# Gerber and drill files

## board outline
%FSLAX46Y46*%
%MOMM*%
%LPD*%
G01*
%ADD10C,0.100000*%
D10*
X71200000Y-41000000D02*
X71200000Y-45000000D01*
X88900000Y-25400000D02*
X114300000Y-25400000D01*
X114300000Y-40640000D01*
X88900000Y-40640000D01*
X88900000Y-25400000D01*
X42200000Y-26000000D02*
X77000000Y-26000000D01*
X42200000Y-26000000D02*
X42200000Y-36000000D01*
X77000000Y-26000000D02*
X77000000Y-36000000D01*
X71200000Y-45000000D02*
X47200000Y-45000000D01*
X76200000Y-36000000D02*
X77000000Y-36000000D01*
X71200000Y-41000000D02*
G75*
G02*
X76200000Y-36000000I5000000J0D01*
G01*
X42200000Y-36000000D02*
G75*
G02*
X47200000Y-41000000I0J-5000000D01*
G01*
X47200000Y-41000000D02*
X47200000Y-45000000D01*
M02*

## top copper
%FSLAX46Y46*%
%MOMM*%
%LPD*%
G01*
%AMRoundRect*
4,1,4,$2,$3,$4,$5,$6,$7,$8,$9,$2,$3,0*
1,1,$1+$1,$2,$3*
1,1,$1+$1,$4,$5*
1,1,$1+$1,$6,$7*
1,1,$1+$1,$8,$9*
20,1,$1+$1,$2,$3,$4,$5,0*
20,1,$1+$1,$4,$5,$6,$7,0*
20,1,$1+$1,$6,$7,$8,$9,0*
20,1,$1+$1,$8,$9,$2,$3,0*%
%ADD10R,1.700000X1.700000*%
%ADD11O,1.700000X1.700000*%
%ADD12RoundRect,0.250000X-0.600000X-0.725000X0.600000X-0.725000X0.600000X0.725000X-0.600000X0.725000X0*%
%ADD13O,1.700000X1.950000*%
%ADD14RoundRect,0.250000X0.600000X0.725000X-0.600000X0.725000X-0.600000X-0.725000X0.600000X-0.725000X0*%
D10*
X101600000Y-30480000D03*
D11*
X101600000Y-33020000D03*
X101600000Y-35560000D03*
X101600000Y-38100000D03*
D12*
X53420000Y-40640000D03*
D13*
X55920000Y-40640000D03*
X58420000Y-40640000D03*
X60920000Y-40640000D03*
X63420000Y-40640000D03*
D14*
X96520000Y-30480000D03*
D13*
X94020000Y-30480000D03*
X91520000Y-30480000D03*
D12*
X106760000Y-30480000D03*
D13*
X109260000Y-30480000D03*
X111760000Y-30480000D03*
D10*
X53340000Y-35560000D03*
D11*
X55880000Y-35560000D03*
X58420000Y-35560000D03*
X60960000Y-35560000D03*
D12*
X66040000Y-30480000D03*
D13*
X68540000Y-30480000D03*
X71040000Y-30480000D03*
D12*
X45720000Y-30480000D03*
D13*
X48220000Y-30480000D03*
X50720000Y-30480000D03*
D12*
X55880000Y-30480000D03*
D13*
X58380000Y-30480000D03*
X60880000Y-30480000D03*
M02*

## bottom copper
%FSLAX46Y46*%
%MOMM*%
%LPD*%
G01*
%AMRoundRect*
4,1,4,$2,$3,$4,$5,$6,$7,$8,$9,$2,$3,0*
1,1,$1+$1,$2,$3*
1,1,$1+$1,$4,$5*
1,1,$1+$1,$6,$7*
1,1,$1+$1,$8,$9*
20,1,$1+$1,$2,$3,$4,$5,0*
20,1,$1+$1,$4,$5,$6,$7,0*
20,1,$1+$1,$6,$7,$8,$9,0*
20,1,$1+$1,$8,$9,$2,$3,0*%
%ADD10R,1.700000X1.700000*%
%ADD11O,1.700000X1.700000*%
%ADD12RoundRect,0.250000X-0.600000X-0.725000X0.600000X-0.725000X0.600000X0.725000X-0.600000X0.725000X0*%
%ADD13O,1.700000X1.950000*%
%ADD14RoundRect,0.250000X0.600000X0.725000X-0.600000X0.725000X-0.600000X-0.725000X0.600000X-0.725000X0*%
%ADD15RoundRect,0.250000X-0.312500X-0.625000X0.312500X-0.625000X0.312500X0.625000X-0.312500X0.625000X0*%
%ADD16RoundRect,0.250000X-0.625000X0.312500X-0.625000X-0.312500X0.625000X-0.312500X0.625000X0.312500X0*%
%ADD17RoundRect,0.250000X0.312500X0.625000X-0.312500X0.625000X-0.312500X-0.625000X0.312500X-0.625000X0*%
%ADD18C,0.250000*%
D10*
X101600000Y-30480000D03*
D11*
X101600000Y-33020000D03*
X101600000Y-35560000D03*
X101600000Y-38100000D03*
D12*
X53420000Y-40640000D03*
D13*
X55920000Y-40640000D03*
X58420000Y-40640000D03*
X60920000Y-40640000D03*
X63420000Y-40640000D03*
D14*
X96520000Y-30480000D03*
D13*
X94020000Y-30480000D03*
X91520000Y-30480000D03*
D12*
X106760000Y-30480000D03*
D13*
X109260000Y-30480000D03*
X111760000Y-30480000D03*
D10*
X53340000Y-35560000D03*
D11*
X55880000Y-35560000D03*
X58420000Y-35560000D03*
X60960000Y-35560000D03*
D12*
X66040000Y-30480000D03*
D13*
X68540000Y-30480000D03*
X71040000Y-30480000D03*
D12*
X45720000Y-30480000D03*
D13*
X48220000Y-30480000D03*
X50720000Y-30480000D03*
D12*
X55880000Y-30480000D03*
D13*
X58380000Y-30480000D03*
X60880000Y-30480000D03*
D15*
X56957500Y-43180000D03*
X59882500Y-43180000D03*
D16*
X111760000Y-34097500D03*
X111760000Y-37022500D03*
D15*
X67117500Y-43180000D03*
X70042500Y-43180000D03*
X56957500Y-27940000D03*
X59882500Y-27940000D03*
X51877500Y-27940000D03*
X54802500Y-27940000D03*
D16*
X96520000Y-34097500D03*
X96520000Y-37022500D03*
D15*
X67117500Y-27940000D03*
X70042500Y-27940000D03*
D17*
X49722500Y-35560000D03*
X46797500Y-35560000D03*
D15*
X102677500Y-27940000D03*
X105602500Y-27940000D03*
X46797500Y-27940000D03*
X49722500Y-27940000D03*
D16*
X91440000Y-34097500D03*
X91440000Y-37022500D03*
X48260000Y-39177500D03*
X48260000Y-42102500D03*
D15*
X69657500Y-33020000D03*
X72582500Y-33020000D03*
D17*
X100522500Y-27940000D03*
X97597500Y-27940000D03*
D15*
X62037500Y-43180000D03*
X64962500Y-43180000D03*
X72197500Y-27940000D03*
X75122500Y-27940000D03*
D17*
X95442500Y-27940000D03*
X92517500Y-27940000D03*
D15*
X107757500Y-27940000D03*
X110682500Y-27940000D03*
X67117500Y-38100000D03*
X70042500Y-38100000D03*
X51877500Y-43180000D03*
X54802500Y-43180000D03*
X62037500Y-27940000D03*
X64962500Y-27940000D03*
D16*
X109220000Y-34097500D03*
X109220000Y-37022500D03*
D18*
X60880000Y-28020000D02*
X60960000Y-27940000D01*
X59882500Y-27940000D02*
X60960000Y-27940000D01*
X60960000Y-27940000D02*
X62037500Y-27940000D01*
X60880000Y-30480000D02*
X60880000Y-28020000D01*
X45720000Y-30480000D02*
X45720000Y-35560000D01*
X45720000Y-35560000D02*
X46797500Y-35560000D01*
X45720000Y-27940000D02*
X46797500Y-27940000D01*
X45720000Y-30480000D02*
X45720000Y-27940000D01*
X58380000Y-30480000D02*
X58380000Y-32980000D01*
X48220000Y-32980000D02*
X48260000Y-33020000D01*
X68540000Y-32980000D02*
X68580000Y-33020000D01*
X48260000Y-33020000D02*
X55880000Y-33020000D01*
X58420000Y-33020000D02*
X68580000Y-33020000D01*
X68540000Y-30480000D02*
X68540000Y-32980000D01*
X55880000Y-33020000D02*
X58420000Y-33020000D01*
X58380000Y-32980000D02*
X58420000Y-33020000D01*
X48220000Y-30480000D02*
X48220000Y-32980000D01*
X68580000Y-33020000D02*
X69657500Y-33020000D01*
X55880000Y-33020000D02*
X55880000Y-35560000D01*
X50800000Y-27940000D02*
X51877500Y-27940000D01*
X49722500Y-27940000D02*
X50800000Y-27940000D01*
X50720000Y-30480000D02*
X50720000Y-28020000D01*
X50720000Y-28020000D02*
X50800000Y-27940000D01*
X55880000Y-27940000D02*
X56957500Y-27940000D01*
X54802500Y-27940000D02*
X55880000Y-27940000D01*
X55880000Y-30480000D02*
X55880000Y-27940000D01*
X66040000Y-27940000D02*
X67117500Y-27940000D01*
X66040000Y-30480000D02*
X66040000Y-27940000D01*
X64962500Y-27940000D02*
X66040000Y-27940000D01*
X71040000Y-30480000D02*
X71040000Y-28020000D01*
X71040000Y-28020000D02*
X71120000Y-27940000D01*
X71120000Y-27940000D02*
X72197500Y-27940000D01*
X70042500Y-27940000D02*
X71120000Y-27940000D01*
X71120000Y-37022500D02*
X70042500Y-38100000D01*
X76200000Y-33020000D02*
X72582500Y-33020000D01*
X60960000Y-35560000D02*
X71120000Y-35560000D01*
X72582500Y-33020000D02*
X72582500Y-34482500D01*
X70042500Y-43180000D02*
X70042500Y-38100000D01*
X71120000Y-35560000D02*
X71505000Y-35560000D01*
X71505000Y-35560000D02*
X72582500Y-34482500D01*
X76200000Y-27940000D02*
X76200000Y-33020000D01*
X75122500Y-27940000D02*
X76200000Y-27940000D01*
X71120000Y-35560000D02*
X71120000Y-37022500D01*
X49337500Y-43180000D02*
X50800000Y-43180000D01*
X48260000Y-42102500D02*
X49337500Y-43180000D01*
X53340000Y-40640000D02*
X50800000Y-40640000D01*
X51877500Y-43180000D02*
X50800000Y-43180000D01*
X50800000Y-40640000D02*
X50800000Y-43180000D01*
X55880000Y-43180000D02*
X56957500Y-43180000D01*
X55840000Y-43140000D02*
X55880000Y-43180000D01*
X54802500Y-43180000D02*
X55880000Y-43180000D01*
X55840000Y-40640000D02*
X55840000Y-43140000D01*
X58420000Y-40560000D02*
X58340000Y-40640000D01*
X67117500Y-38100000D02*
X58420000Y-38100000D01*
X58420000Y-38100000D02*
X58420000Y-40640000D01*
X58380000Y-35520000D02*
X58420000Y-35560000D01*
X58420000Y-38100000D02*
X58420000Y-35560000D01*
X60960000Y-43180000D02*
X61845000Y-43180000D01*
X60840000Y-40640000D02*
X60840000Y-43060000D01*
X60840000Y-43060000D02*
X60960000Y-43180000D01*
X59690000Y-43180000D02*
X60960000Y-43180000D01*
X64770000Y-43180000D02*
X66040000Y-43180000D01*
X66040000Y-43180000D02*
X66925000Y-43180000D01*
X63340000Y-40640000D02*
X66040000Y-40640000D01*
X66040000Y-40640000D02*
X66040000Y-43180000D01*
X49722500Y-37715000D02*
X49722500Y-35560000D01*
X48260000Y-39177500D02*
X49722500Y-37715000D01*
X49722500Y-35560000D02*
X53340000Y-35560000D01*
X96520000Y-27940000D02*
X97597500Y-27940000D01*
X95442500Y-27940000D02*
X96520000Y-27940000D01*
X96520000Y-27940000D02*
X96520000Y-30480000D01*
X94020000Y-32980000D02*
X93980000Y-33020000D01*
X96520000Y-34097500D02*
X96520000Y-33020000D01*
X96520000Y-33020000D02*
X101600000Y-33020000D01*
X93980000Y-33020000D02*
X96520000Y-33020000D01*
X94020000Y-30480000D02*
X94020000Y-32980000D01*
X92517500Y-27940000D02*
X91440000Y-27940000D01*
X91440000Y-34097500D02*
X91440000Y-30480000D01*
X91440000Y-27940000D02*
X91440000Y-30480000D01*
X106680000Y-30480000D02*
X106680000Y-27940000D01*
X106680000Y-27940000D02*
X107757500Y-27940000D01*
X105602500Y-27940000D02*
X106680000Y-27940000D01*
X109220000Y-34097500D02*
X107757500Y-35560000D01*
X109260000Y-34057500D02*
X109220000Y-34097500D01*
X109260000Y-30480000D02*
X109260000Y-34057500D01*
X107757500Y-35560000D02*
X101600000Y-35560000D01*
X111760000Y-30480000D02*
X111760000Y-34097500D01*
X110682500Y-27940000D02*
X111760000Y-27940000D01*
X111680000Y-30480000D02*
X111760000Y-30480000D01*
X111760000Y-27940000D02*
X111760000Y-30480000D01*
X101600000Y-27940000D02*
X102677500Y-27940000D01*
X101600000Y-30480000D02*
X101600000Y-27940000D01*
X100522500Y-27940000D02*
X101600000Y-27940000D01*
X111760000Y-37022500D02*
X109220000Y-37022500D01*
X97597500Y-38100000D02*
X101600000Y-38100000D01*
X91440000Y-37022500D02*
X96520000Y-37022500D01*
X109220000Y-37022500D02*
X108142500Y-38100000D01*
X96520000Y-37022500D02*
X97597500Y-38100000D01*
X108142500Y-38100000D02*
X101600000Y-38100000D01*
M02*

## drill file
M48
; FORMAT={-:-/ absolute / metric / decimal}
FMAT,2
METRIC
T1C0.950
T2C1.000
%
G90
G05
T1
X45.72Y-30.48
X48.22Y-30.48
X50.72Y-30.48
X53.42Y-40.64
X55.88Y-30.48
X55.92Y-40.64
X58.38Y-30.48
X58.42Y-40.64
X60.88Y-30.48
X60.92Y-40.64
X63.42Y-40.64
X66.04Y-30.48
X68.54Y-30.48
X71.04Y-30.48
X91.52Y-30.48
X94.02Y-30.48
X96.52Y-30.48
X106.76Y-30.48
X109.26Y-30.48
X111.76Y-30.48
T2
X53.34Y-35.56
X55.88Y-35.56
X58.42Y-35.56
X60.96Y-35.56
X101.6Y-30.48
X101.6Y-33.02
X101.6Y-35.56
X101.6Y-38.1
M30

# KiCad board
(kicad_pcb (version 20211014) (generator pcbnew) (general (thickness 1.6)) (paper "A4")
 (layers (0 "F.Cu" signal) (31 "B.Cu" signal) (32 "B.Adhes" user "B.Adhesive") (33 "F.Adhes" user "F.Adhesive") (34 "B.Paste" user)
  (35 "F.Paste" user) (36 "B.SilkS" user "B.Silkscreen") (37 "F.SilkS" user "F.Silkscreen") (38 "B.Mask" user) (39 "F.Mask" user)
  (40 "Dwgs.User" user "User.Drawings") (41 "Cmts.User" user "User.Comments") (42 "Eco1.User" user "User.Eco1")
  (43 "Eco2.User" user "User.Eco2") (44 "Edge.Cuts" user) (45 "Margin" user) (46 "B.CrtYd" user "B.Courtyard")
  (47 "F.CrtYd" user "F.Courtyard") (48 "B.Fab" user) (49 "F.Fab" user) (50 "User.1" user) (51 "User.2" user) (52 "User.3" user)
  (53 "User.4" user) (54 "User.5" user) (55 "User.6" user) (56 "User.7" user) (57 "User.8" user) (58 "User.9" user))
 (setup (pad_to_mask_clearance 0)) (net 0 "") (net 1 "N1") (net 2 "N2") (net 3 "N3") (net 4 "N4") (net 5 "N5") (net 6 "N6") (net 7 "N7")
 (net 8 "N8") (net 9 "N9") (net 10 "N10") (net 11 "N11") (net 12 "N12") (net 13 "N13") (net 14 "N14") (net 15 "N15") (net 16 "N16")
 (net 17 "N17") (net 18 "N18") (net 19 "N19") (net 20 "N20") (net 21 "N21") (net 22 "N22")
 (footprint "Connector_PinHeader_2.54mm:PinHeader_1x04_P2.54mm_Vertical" (layer "F.Cu") (at 101.6 30.48)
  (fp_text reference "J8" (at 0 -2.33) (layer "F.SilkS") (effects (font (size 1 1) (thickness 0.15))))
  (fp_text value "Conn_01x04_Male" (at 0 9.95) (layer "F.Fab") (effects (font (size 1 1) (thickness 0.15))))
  (pad "1" thru_hole rect (at 0 0) (size 1.7 1.7) (drill 1) (layers *.Cu *.Mask) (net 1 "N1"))
  (pad "2" thru_hole oval (at 0 2.54) (size 1.7 1.7) (drill 1) (layers *.Cu *.Mask) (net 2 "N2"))
  (pad "3" thru_hole oval (at 0 5.08) (size 1.7 1.7) (drill 1) (layers *.Cu *.Mask) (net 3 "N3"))
  (pad "4" thru_hole oval (at 0 7.62) (size 1.7 1.7) (drill 1) (layers *.Cu *.Mask) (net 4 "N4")))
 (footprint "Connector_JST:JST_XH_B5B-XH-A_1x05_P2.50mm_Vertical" (layer "F.Cu") (at 53.42 40.64)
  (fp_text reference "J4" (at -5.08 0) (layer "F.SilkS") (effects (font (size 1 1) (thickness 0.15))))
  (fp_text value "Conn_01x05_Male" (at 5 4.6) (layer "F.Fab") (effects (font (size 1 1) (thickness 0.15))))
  (pad "1" thru_hole roundrect (at 0 0) (size 1.7 1.95) (drill 0.95) (layers *.Cu *.Mask) (roundrect_rratio 0.1470588235) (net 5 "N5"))
  (pad "2" thru_hole oval (at 2.5 0) (size 1.7 1.95) (drill 0.95) (layers *.Cu *.Mask) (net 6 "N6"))
  (pad "3" thru_hole oval (at 5 0) (size 1.7 1.95) (drill 0.95) (layers *.Cu *.Mask) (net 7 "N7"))
  (pad "4" thru_hole oval (at 7.5 0) (size 1.7 1.95) (drill 0.95) (layers *.Cu *.Mask) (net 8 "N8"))
  (pad "5" thru_hole oval (at 10 0) (size 1.7 1.95) (drill 0.95) (layers *.Cu *.Mask) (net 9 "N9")))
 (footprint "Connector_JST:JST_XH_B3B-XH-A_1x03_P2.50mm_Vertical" (layer "F.Cu") (at 96.52 30.48 180)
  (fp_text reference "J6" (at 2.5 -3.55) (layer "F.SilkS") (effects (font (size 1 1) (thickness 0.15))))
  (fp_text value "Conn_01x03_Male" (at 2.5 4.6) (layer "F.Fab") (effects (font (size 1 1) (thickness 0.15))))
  (pad "1" thru_hole roundrect (at 0 0 180) (size 1.7 1.95) (drill 0.95) (layers *.Cu *.Mask) (roundrect_rratio 0.1470588235) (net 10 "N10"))
  (pad "2" thru_hole oval (at 2.5 0 180) (size 1.7 1.95) (drill 0.95) (layers *.Cu *.Mask) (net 2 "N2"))
  (pad "3" thru_hole oval (at 5 0 180) (size 1.7 1.95) (drill 0.95) (layers *.Cu *.Mask) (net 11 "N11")))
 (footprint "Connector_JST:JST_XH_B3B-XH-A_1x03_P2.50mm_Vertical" (layer "F.Cu") (at 106.76 30.48)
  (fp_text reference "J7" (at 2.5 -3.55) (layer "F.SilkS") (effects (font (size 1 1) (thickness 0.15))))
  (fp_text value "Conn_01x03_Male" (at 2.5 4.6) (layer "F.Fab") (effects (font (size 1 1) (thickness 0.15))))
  (pad "1" thru_hole roundrect (at 0 0) (size 1.7 1.95) (drill 0.95) (layers *.Cu *.Mask) (roundrect_rratio 0.1470588235) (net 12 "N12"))
  (pad "2" thru_hole oval (at 2.5 0) (size 1.7 1.95) (drill 0.95) (layers *.Cu *.Mask) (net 3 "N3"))
  (pad "3" thru_hole oval (at 5 0) (size 1.7 1.95) (drill 0.95) (layers *.Cu *.Mask) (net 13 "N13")))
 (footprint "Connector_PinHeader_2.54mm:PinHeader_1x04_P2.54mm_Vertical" (layer "F.Cu") (at 53.34 35.56 90)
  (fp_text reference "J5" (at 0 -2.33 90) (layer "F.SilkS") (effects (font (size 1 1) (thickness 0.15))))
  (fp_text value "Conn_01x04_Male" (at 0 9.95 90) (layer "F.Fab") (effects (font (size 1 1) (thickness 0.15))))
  (pad "1" thru_hole rect (at 0 0 90) (size 1.7 1.7) (drill 1) (layers *.Cu *.Mask) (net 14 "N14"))
  (pad "2" thru_hole oval (at 0 2.54 90) (size 1.7 1.7) (drill 1) (layers *.Cu *.Mask) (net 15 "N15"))
  (pad "3" thru_hole oval (at 0 5.08 90) (size 1.7 1.7) (drill 1) (layers *.Cu *.Mask) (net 7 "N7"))
  (pad "4" thru_hole oval (at 0 7.62 90) (size 1.7 1.7) (drill 1) (layers *.Cu *.Mask) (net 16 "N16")))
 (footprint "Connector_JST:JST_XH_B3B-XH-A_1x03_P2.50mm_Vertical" (layer "F.Cu") (at 66.04 30.48)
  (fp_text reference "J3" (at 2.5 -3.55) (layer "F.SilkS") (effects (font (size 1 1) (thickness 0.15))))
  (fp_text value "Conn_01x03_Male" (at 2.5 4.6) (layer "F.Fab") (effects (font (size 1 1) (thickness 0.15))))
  (pad "1" thru_hole roundrect (at 0 0) (size 1.7 1.95) (drill 0.95) (layers *.Cu *.Mask) (roundrect_rratio 0.1470588235) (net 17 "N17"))
  (pad "2" thru_hole oval (at 2.5 0) (size 1.7 1.95) (drill 0.95) (layers *.Cu *.Mask) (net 15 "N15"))
  (pad "3" thru_hole oval (at 5 0) (size 1.7 1.95) (drill 0.95) (layers *.Cu *.Mask) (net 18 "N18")))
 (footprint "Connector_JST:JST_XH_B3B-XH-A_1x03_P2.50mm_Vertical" (layer "F.Cu") (at 45.72 30.48)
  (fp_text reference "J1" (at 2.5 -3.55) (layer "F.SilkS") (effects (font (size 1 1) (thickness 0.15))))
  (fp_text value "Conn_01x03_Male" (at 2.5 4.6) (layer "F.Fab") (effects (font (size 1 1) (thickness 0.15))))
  (pad "1" thru_hole roundrect (at 0 0) (size 1.7 1.95) (drill 0.95) (layers *.Cu *.Mask) (roundrect_rratio 0.1470588235) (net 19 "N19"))
  (pad "2" thru_hole oval (at 2.5 0) (size 1.7 1.95) (drill 0.95) (layers *.Cu *.Mask) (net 15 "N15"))
  (pad "3" thru_hole oval (at 5 0) (size 1.7 1.95) (drill 0.95) (layers *.Cu *.Mask) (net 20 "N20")))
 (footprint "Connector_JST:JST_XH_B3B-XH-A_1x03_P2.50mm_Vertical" (layer "F.Cu") (at 55.88 30.48)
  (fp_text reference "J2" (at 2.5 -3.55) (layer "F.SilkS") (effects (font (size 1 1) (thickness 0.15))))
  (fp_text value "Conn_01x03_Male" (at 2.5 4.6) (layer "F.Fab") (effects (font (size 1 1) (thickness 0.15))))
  (pad "1" thru_hole roundrect (at 0 0) (size 1.7 1.95) (drill 0.95) (layers *.Cu *.Mask) (roundrect_rratio 0.1470588235) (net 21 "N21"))
  (pad "2" thru_hole oval (at 2.5 0) (size 1.7 1.95) (drill 0.95) (layers *.Cu *.Mask) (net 15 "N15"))
  (pad "3" thru_hole oval (at 5 0) (size 1.7 1.95) (drill 0.95) (layers *.Cu *.Mask) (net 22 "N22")))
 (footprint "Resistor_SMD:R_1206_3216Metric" (layer "B.Cu") (at 58.42 43.18)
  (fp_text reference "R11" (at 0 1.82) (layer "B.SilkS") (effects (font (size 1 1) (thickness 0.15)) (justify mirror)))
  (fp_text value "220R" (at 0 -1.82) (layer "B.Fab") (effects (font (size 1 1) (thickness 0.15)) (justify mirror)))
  (pad "1" smd roundrect (at -1.4625 0) (size 1.125 1.75) (layers "B.Cu" "B.Paste" "B.Mask") (roundrect_rratio 0.2222222222) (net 6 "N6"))
  (pad "2" smd roundrect (at 1.4625 0) (size 1.125 1.75) (layers "B.Cu" "B.Paste" "B.Mask") (roundrect_rratio 0.2222222222) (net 8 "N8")))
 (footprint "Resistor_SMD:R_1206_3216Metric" (layer "B.Cu") (at 111.76 35.56 -90)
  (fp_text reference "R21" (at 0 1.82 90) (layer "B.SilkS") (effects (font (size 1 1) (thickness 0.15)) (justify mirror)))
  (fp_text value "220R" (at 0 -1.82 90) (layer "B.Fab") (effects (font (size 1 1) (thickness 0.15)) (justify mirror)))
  (pad "1" smd roundrect (at -1.4625 0 270) (size 1.125 1.75) (layers "B.Cu" "B.Paste" "B.Mask") (roundrect_rratio 0.2222222222)
   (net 13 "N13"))
  (pad "2" smd roundrect (at 1.4625 0 270) (size 1.125 1.75) (layers "B.Cu" "B.Paste" "B.Mask") (roundrect_rratio 0.2222222222) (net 4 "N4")))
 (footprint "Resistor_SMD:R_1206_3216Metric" (layer "B.Cu") (at 68.58 43.18)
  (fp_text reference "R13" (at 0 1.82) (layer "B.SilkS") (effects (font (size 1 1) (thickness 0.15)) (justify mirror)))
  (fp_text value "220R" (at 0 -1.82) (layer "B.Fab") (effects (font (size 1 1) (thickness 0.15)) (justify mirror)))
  (pad "1" smd roundrect (at -1.4625 0) (size 1.125 1.75) (layers "B.Cu" "B.Paste" "B.Mask") (roundrect_rratio 0.2222222222) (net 9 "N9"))
  (pad "2" smd roundrect (at 1.4625 0) (size 1.125 1.75) (layers "B.Cu" "B.Paste" "B.Mask") (roundrect_rratio 0.2222222222) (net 16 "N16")))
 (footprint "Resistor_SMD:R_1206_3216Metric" (layer "B.Cu") (at 58.42 27.94)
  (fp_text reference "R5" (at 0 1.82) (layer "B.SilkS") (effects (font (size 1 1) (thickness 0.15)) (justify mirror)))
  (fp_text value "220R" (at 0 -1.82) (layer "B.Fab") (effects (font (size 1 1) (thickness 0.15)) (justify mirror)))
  (pad "1" smd roundrect (at -1.4625 0) (size 1.125 1.75) (layers "B.Cu" "B.Paste" "B.Mask") (roundrect_rratio 0.2222222222) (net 21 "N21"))
  (pad "2" smd roundrect (at 1.4625 0) (size 1.125 1.75) (layers "B.Cu" "B.Paste" "B.Mask") (roundrect_rratio 0.2222222222) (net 22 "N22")))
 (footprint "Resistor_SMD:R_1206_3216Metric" (layer "B.Cu") (at 53.34 27.94)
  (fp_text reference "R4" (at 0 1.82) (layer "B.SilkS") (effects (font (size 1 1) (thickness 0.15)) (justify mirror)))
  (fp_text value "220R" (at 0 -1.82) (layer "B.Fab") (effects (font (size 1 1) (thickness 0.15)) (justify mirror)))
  (pad "1" smd roundrect (at -1.4625 0) (size 1.125 1.75) (layers "B.Cu" "B.Paste" "B.Mask") (roundrect_rratio 0.2222222222) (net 20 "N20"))
  (pad "2" smd roundrect (at 1.4625 0) (size 1.125 1.75) (layers "B.Cu" "B.Paste" "B.Mask") (roundrect_rratio 0.2222222222) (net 21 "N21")))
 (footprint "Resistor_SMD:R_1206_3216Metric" (layer "B.Cu") (at 96.52 35.56 -90)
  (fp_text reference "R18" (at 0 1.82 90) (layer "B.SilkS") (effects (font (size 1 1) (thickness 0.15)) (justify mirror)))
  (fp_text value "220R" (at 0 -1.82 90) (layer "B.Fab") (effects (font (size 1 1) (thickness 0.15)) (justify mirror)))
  (pad "1" smd roundrect (at -1.4625 0 270) (size 1.125 1.75) (layers "B.Cu" "B.Paste" "B.Mask") (roundrect_rratio 0.2222222222)
   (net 2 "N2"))
  (pad "2" smd roundrect (at 1.4625 0 270) (size 1.125 1.75) (layers "B.Cu" "B.Paste" "B.Mask") (roundrect_rratio 0.2222222222) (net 4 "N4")))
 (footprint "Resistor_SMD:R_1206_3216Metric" (layer "B.Cu") (at 68.58 27.94)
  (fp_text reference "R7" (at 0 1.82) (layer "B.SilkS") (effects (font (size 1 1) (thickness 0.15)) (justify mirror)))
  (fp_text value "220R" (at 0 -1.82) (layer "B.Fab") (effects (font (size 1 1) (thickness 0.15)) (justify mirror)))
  (pad "1" smd roundrect (at -1.4625 0) (size 1.125 1.75) (layers "B.Cu" "B.Paste" "B.Mask") (roundrect_rratio 0.2222222222) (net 17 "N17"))
  (pad "2" smd roundrect (at 1.4625 0) (size 1.125 1.75) (layers "B.Cu" "B.Paste" "B.Mask") (roundrect_rratio 0.2222222222) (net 18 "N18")))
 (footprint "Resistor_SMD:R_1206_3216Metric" (layer "B.Cu") (at 48.26 35.56 180)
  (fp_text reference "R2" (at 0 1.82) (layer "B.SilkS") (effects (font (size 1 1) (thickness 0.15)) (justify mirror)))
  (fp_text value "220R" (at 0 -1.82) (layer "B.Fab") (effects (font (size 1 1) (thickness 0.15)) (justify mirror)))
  (pad "1" smd roundrect (at -1.4625 0 180) (size 1.125 1.75) (layers "B.Cu" "B.Paste" "B.Mask") (roundrect_rratio 0.2222222222)
   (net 14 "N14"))
  (pad "2" smd roundrect (at 1.4625 0 180) (size 1.125 1.75) (layers "B.Cu" "B.Paste" "B.Mask") (roundrect_rratio 0.2222222222)
   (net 19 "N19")))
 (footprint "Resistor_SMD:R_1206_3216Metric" (layer "B.Cu") (at 104.14 27.94)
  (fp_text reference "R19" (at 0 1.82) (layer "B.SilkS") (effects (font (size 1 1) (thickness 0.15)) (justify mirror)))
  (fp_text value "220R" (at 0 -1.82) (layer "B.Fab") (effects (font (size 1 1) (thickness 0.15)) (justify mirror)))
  (pad "1" smd roundrect (at -1.4625 0) (size 1.125 1.75) (layers "B.Cu" "B.Paste" "B.Mask") (roundrect_rratio 0.2222222222) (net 1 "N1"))
  (pad "2" smd roundrect (at 1.4625 0) (size 1.125 1.75) (layers "B.Cu" "B.Paste" "B.Mask") (roundrect_rratio 0.2222222222) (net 12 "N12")))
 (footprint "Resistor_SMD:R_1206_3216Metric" (layer "B.Cu") (at 48.26 27.94)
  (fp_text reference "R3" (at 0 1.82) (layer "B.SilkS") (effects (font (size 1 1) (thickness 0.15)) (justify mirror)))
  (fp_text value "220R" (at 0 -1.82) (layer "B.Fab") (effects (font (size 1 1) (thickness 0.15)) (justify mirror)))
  (pad "1" smd roundrect (at -1.4625 0) (size 1.125 1.75) (layers "B.Cu" "B.Paste" "B.Mask") (roundrect_rratio 0.2222222222) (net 19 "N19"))
  (pad "2" smd roundrect (at 1.4625 0) (size 1.125 1.75) (layers "B.Cu" "B.Paste" "B.Mask") (roundrect_rratio 0.2222222222) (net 20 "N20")))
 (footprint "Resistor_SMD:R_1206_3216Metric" (layer "B.Cu") (at 91.44 35.56 -90)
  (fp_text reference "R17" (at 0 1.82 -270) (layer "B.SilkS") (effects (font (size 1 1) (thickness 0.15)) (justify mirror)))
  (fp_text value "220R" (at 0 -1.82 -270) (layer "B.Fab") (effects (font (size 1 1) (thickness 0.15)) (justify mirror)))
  (pad "1" smd roundrect (at -1.4625 0 270) (size 1.125 1.75) (layers "B.Cu" "B.Paste" "B.Mask") (roundrect_rratio 0.2222222222)
   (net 11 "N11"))
  (pad "2" smd roundrect (at 1.4625 0 270) (size 1.125 1.75) (layers "B.Cu" "B.Paste" "B.Mask") (roundrect_rratio 0.2222222222) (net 4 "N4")))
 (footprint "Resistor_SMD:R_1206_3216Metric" (layer "B.Cu") (at 48.26 40.64 -90)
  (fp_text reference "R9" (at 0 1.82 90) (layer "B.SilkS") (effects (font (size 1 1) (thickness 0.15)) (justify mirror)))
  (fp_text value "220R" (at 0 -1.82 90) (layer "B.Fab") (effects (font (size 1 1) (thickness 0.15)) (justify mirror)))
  (pad "1" smd roundrect (at -1.4625 0 270) (size 1.125 1.75) (layers "B.Cu" "B.Paste" "B.Mask") (roundrect_rratio 0.2222222222)
   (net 14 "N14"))
  (pad "2" smd roundrect (at 1.4625 0 270) (size 1.125 1.75) (layers "B.Cu" "B.Paste" "B.Mask") (roundrect_rratio 0.2222222222) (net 5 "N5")))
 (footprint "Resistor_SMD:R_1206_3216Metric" (layer "B.Cu") (at 71.12 33.02)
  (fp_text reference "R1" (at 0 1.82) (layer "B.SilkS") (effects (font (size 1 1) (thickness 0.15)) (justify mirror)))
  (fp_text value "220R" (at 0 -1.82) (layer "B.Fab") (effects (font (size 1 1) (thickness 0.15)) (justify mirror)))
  (pad "1" smd roundrect (at -1.4625 0) (size 1.125 1.75) (layers "B.Cu" "B.Paste" "B.Mask") (roundrect_rratio 0.2222222222) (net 15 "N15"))
  (pad "2" smd roundrect (at 1.4625 0) (size 1.125 1.75) (layers "B.Cu" "B.Paste" "B.Mask") (roundrect_rratio 0.2222222222) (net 16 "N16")))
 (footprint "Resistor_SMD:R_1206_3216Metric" (layer "B.Cu") (at 99.06 27.94 180)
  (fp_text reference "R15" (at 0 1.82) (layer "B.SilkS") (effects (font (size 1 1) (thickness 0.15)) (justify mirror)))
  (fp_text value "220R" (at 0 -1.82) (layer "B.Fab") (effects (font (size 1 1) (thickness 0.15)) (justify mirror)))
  (pad "1" smd roundrect (at -1.4625 0 180) (size 1.125 1.75) (layers "B.Cu" "B.Paste" "B.Mask") (roundrect_rratio 0.2222222222)
   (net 1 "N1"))
  (pad "2" smd roundrect (at 1.4625 0 180) (size 1.125 1.75) (layers "B.Cu" "B.Paste" "B.Mask") (roundrect_rratio 0.2222222222)
   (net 10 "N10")))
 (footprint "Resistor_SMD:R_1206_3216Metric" (layer "B.Cu") (at 63.5 43.18)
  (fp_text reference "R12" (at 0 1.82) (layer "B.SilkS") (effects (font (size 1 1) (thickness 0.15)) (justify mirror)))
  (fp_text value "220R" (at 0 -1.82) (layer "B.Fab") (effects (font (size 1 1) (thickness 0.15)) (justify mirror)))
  (pad "1" smd roundrect (at -1.4625 0) (size 1.125 1.75) (layers "B.Cu" "B.Paste" "B.Mask") (roundrect_rratio 0.2222222222) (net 8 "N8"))
  (pad "2" smd roundrect (at 1.4625 0) (size 1.125 1.75) (layers "B.Cu" "B.Paste" "B.Mask") (roundrect_rratio 0.2222222222) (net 9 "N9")))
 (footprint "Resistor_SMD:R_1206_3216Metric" (layer "B.Cu") (at 73.66 27.94)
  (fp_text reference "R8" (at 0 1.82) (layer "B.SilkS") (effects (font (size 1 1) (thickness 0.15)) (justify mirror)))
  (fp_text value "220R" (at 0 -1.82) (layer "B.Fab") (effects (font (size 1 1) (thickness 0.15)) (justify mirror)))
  (pad "1" smd roundrect (at -1.4625 0) (size 1.125 1.75) (layers "B.Cu" "B.Paste" "B.Mask") (roundrect_rratio 0.2222222222) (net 18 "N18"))
  (pad "2" smd roundrect (at 1.4625 0) (size 1.125 1.75) (layers "B.Cu" "B.Paste" "B.Mask") (roundrect_rratio 0.2222222222) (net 16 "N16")))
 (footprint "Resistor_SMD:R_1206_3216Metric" (layer "B.Cu") (at 93.98 27.94 180)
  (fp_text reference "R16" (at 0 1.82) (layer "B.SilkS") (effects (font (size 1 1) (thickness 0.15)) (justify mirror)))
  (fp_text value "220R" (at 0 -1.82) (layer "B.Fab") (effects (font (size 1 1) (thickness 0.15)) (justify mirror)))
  (pad "1" smd roundrect (at -1.4625 0 180) (size 1.125 1.75) (layers "B.Cu" "B.Paste" "B.Mask") (roundrect_rratio 0.2222222222)
   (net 10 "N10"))
  (pad "2" smd roundrect (at 1.4625 0 180) (size 1.125 1.75) (layers "B.Cu" "B.Paste" "B.Mask") (roundrect_rratio 0.2222222222)
   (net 11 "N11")))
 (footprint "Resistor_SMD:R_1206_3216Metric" (layer "B.Cu") (at 109.22 27.94)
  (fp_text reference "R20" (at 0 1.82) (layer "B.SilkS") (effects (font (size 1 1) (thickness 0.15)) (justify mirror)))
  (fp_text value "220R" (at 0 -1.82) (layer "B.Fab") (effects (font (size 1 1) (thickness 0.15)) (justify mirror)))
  (pad "1" smd roundrect (at -1.4625 0) (size 1.125 1.75) (layers "B.Cu" "B.Paste" "B.Mask") (roundrect_rratio 0.2222222222) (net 12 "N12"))
  (pad "2" smd roundrect (at 1.4625 0) (size 1.125 1.75) (layers "B.Cu" "B.Paste" "B.Mask") (roundrect_rratio 0.2222222222) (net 13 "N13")))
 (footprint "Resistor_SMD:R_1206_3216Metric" (layer "B.Cu") (at 68.58 38.1)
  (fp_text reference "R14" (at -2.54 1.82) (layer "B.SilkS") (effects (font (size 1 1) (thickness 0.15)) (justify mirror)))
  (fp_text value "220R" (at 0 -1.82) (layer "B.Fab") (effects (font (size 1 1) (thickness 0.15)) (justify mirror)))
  (pad "1" smd roundrect (at -1.4625 0) (size 1.125 1.75) (layers "B.Cu" "B.Paste" "B.Mask") (roundrect_rratio 0.2222222222) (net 7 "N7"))
  (pad "2" smd roundrect (at 1.4625 0) (size 1.125 1.75) (layers "B.Cu" "B.Paste" "B.Mask") (roundrect_rratio 0.2222222222) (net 16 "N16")))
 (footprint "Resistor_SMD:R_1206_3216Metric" (layer "B.Cu") (at 53.34 43.18)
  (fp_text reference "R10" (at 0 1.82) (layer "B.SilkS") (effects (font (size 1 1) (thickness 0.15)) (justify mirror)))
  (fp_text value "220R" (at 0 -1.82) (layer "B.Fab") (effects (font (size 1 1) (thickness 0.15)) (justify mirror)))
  (pad "1" smd roundrect (at -1.4625 0) (size 1.125 1.75) (layers "B.Cu" "B.Paste" "B.Mask") (roundrect_rratio 0.2222222222) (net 5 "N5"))
  (pad "2" smd roundrect (at 1.4625 0) (size 1.125 1.75) (layers "B.Cu" "B.Paste" "B.Mask") (roundrect_rratio 0.2222222222) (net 6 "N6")))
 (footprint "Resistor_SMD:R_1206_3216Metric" (layer "B.Cu") (at 63.5 27.94)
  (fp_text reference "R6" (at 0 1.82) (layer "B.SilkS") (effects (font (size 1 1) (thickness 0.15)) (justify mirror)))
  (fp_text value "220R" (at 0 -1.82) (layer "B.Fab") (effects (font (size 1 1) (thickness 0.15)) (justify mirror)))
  (pad "1" smd roundrect (at -1.4625 0) (size 1.125 1.75) (layers "B.Cu" "B.Paste" "B.Mask") (roundrect_rratio 0.2222222222) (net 22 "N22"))
  (pad "2" smd roundrect (at 1.4625 0) (size 1.125 1.75) (layers "B.Cu" "B.Paste" "B.Mask") (roundrect_rratio 0.2222222222) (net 17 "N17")))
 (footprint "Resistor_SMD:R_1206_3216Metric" (layer "B.Cu") (at 109.22 35.56 -90)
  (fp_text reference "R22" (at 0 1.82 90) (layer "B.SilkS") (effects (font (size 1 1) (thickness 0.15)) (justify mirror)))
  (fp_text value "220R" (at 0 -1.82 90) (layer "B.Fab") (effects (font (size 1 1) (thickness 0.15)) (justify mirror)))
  (pad "1" smd roundrect (at -1.4625 0 270) (size 1.125 1.75) (layers "B.Cu" "B.Paste" "B.Mask") (roundrect_rratio 0.2222222222)
   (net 3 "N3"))
  (pad "2" smd roundrect (at 1.4625 0 270) (size 1.125 1.75) (layers "B.Cu" "B.Paste" "B.Mask") (roundrect_rratio 0.2222222222) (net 4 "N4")))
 (gr_line (start 71.2 41) (end 71.2 45) (layer "Edge.Cuts") (width 0.1))
 (gr_rect (start 88.9 25.4) (end 114.3 40.64) (layer "Edge.Cuts") (width 0.1) (fill none))
 (gr_line (start 42.2 26) (end 77 26) (layer "Edge.Cuts") (width 0.1))
 (gr_line (start 42.2 26) (end 42.2 36) (layer "Edge.Cuts") (width 0.1))
 (gr_line (start 77 26) (end 77 36) (layer "Edge.Cuts") (width 0.1))
 (gr_line (start 71.2 45) (end 47.2 45) (layer "Edge.Cuts") (width 0.1))
 (gr_line (start 76.2 36) (end 77 36) (layer "Edge.Cuts") (width 0.1))
 (gr_arc (start 71.2 41) (mid 72.664466 37.464466) (end 76.2 36) (layer "Edge.Cuts") (width 0.1))
 (gr_arc (start 42.2 36) (mid 45.735534 37.464466) (end 47.2 41) (layer "Edge.Cuts") (width 0.1))
 (gr_line (start 47.2 41) (end 47.2 45) (layer "Edge.Cuts") (width 0.1))
 (segment (start 60.88 28.02) (end 60.96 27.94) (width 0.25) (layer "B.Cu") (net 22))
 (segment (start 59.8825 27.94) (end 60.96 27.94) (width 0.25) (layer "B.Cu") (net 22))
 (segment (start 60.96 27.94) (end 62.0375 27.94) (width 0.25) (layer "B.Cu") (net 22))
 (segment (start 60.88 30.48) (end 60.88 28.02) (width 0.25) (layer "B.Cu") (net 22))
 (segment (start 45.72 30.48) (end 45.72 35.56) (width 0.25) (layer "B.Cu") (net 19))
 (segment (start 45.72 35.56) (end 46.7975 35.56) (width 0.25) (layer "B.Cu") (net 19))
 (segment (start 45.72 27.94) (end 46.7975 27.94) (width 0.25) (layer "B.Cu") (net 19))
 (segment (start 45.72 30.48) (end 45.72 27.94) (width 0.25) (layer "B.Cu") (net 19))
 (segment (start 58.38 30.48) (end 58.38 32.98) (width 0.25) (layer "B.Cu") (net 15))
 (segment (start 48.22 32.98) (end 48.26 33.02) (width 0.25) (layer "B.Cu") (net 15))
 (segment (start 68.54 32.98) (end 68.58 33.02) (width 0.25) (layer "B.Cu") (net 15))
 (segment (start 48.26 33.02) (end 55.88 33.02) (width 0.25) (layer "B.Cu") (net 15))
 (segment (start 58.42 33.02) (end 68.58 33.02) (width 0.25) (layer "B.Cu") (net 15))
 (segment (start 68.54 30.48) (end 68.54 32.98) (width 0.25) (layer "B.Cu") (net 15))
 (segment (start 55.88 33.02) (end 58.42 33.02) (width 0.25) (layer "B.Cu") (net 15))
 (segment (start 58.38 32.98) (end 58.42 33.02) (width 0.25) (layer "B.Cu") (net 15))
 (segment (start 48.22 30.48) (end 48.22 32.98) (width 0.25) (layer "B.Cu") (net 15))
 (segment (start 68.58 33.02) (end 69.6575 33.02) (width 0.25) (layer "B.Cu") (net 15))
 (segment (start 55.88 33.02) (end 55.88 35.56) (width 0.25) (layer "B.Cu") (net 15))
 (segment (start 50.8 27.94) (end 51.8775 27.94) (width 0.25) (layer "B.Cu") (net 20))
 (segment (start 49.7225 27.94) (end 50.8 27.94) (width 0.25) (layer "B.Cu") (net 20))
 (segment (start 50.72 30.48) (end 50.72 28.02) (width 0.25) (layer "B.Cu") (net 20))
 (segment (start 50.72 28.02) (end 50.8 27.94) (width 0.25) (layer "B.Cu") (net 20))
 (segment (start 55.88 27.94) (end 56.9575 27.94) (width 0.25) (layer "B.Cu") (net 21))
 (segment (start 54.8025 27.94) (end 55.88 27.94) (width 0.25) (layer "B.Cu") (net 21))
 (segment (start 55.88 30.48) (end 55.88 27.94) (width 0.25) (layer "B.Cu") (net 21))
 (segment (start 66.04 27.94) (end 67.1175 27.94) (width 0.25) (layer "B.Cu") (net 17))
 (segment (start 66.04 30.48) (end 66.04 27.94) (width 0.25) (layer "B.Cu") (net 17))
 (segment (start 64.9625 27.94) (end 66.04 27.94) (width 0.25) (layer "B.Cu") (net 17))
 (segment (start 71.04 30.48) (end 71.04 28.02) (width 0.25) (layer "B.Cu") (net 18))
 (segment (start 71.04 28.02) (end 71.12 27.94) (width 0.25) (layer "B.Cu") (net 18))
 (segment (start 71.12 27.94) (end 72.1975 27.94) (width 0.25) (layer "B.Cu") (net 18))
 (segment (start 70.0425 27.94) (end 71.12 27.94) (width 0.25) (layer "B.Cu") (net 18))
 (segment (start 71.12 37.0225) (end 70.0425 38.1) (width 0.25) (layer "B.Cu") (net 16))
 (segment (start 76.2 33.02) (end 72.5825 33.02) (width 0.25) (layer "B.Cu") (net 16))
 (segment (start 60.96 35.56) (end 71.12 35.56) (width 0.25) (layer "B.Cu") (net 16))
 (segment (start 72.5825 33.02) (end 72.5825 34.4825) (width 0.25) (layer "B.Cu") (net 16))
 (segment (start 70.0425 43.18) (end 70.0425 38.1) (width 0.25) (layer "B.Cu") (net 16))
 (segment (start 71.12 35.56) (end 71.505 35.56) (width 0.25) (layer "B.Cu") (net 16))
 (segment (start 71.505 35.56) (end 72.5825 34.4825) (width 0.25) (layer "B.Cu") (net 16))
 (segment (start 76.2 27.94) (end 76.2 33.02) (width 0.25) (layer "B.Cu") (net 16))
 (segment (start 75.1225 27.94) (end 76.2 27.94) (width 0.25) (layer "B.Cu") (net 16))
 (segment (start 71.12 35.56) (end 71.12 37.0225) (width 0.25) (layer "B.Cu") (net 16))
 (segment (start 49.3375 43.18) (end 50.8 43.18) (width 0.25) (layer "B.Cu") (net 5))
 (segment (start 48.26 42.1025) (end 49.3375 43.18) (width 0.25) (layer "B.Cu") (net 5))
 (segment (start 53.34 40.64) (end 50.8 40.64) (width 0.25) (layer "B.Cu") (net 5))
 (segment (start 51.8775 43.18) (end 50.8 43.18) (width 0.25) (layer "B.Cu") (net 5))
 (segment (start 50.8 40.64) (end 50.8 43.18) (width 0.25) (layer "B.Cu") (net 5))
 (segment (start 55.88 43.18) (end 56.9575 43.18) (width 0.25) (layer "B.Cu") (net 6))
 (segment (start 55.84 43.14) (end 55.88 43.18) (width 0.25) (layer "B.Cu") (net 6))
 (segment (start 54.8025 43.18) (end 55.88 43.18) (width 0.25) (layer "B.Cu") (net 6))
 (segment (start 55.84 40.64) (end 55.84 43.14) (width 0.25) (layer "B.Cu") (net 6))
 (segment (start 58.42 40.56) (end 58.34 40.64) (width 0.25) (layer "B.Cu") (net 7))
 (segment (start 67.1175 38.1) (end 58.42 38.1) (width 0.25) (layer "B.Cu") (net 7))
 (segment (start 58.42 38.1) (end 58.42 40.64) (width 0.25) (layer "B.Cu") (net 7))
 (segment (start 58.38 35.52) (end 58.42 35.56) (width 0.25) (layer "B.Cu") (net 7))
 (segment (start 58.42 38.1) (end 58.42 35.56) (width 0.25) (layer "B.Cu") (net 7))
 (segment (start 60.96 43.18) (end 61.845 43.18) (width 0.25) (layer "B.Cu") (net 8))
 (segment (start 60.84 40.64) (end 60.84 43.06) (width 0.25) (layer "B.Cu") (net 8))
 (segment (start 60.84 43.06) (end 60.96 43.18) (width 0.25) (layer "B.Cu") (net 8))
 (segment (start 59.69 43.18) (end 60.96 43.18) (width 0.25) (layer "B.Cu") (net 8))
 (segment (start 64.77 43.18) (end 66.04 43.18) (width 0.25) (layer "B.Cu") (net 9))
 (segment (start 66.04 43.18) (end 66.925 43.18) (width 0.25) (layer "B.Cu") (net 9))
 (segment (start 63.34 40.64) (end 66.04 40.64) (width 0.25) (layer "B.Cu") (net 9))
 (segment (start 66.04 40.64) (end 66.04 43.18) (width 0.25) (layer "B.Cu") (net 9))
 (segment (start 49.7225 37.715) (end 49.7225 35.56) (width 0.25) (layer "B.Cu") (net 14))
 (segment (start 48.26 39.1775) (end 49.7225 37.715) (width 0.25) (layer "B.Cu") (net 14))
 (segment (start 49.7225 35.56) (end 53.34 35.56) (width 0.25) (layer "B.Cu") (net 14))
 (segment (start 96.52 27.94) (end 97.5975 27.94) (width 0.25) (layer "B.Cu") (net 10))
 (segment (start 95.4425 27.94) (end 96.52 27.94) (width 0.25) (layer "B.Cu") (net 10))
 (segment (start 96.52 27.94) (end 96.52 30.48) (width 0.25) (layer "B.Cu") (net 10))
 (segment (start 94.02 32.98) (end 93.98 33.02) (width 0.25) (layer "B.Cu") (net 2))
 (segment (start 96.52 34.0975) (end 96.52 33.02) (width 0.25) (layer "B.Cu") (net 2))
 (segment (start 96.52 33.02) (end 101.6 33.02) (width 0.25) (layer "B.Cu") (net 2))
 (segment (start 93.98 33.02) (end 96.52 33.02) (width 0.25) (layer "B.Cu") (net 2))
 (segment (start 94.02 30.48) (end 94.02 32.98) (width 0.25) (layer "B.Cu") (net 2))
 (segment (start 92.5175 27.94) (end 91.44 27.94) (width 0.25) (layer "B.Cu") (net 11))
 (segment (start 91.44 34.0975) (end 91.44 30.48) (width 0.25) (layer "B.Cu") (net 11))
 (segment (start 91.44 27.94) (end 91.44 30.48) (width 0.25) (layer "B.Cu") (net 11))
 (segment (start 106.68 30.48) (end 106.68 27.94) (width 0.25) (layer "B.Cu") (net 12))
 (segment (start 106.68 27.94) (end 107.7575 27.94) (width 0.25) (layer "B.Cu") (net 12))
 (segment (start 105.6025 27.94) (end 106.68 27.94) (width 0.25) (layer "B.Cu") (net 12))
 (segment (start 109.22 34.0975) (end 107.7575 35.56) (width 0.25) (layer "B.Cu") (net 3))
 (segment (start 109.26 34.0575) (end 109.22 34.0975) (width 0.25) (layer "B.Cu") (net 3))
 (segment (start 109.26 30.48) (end 109.26 34.0575) (width 0.25) (layer "B.Cu") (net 3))
 (segment (start 107.7575 35.56) (end 101.6 35.56) (width 0.25) (layer "B.Cu") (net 3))
 (segment (start 111.76 30.48) (end 111.76 34.0975) (width 0.25) (layer "B.Cu") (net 13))
 (segment (start 110.6825 27.94) (end 111.76 27.94) (width 0.25) (layer "B.Cu") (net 13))
 (segment (start 111.68 30.48) (end 111.76 30.48) (width 0.25) (layer "B.Cu") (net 13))
 (segment (start 111.76 27.94) (end 111.76 30.48) (width 0.25) (layer "B.Cu") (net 13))
 (segment (start 101.6 27.94) (end 102.6775 27.94) (width 0.25) (layer "B.Cu") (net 1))
 (segment (start 101.6 30.48) (end 101.6 27.94) (width 0.25) (layer "B.Cu") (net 1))
 (segment (start 100.5225 27.94) (end 101.6 27.94) (width 0.25) (layer "B.Cu") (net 1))
 (segment (start 111.76 37.0225) (end 109.22 37.0225) (width 0.25) (layer "B.Cu") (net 4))
 (segment (start 97.5975 38.1) (end 101.6 38.1) (width 0.25) (layer "B.Cu") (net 4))
 (segment (start 91.44 37.0225) (end 96.52 37.0225) (width 0.25) (layer "B.Cu") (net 4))
 (segment (start 109.22 37.0225) (end 108.1425 38.1) (width 0.25) (layer "B.Cu") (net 4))
 (segment (start 96.52 37.0225) (end 97.5975 38.1) (width 0.25) (layer "B.Cu") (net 4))
 (segment (start 108.1425 38.1) (end 101.6 38.1) (width 0.25) (layer "B.Cu") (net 4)))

